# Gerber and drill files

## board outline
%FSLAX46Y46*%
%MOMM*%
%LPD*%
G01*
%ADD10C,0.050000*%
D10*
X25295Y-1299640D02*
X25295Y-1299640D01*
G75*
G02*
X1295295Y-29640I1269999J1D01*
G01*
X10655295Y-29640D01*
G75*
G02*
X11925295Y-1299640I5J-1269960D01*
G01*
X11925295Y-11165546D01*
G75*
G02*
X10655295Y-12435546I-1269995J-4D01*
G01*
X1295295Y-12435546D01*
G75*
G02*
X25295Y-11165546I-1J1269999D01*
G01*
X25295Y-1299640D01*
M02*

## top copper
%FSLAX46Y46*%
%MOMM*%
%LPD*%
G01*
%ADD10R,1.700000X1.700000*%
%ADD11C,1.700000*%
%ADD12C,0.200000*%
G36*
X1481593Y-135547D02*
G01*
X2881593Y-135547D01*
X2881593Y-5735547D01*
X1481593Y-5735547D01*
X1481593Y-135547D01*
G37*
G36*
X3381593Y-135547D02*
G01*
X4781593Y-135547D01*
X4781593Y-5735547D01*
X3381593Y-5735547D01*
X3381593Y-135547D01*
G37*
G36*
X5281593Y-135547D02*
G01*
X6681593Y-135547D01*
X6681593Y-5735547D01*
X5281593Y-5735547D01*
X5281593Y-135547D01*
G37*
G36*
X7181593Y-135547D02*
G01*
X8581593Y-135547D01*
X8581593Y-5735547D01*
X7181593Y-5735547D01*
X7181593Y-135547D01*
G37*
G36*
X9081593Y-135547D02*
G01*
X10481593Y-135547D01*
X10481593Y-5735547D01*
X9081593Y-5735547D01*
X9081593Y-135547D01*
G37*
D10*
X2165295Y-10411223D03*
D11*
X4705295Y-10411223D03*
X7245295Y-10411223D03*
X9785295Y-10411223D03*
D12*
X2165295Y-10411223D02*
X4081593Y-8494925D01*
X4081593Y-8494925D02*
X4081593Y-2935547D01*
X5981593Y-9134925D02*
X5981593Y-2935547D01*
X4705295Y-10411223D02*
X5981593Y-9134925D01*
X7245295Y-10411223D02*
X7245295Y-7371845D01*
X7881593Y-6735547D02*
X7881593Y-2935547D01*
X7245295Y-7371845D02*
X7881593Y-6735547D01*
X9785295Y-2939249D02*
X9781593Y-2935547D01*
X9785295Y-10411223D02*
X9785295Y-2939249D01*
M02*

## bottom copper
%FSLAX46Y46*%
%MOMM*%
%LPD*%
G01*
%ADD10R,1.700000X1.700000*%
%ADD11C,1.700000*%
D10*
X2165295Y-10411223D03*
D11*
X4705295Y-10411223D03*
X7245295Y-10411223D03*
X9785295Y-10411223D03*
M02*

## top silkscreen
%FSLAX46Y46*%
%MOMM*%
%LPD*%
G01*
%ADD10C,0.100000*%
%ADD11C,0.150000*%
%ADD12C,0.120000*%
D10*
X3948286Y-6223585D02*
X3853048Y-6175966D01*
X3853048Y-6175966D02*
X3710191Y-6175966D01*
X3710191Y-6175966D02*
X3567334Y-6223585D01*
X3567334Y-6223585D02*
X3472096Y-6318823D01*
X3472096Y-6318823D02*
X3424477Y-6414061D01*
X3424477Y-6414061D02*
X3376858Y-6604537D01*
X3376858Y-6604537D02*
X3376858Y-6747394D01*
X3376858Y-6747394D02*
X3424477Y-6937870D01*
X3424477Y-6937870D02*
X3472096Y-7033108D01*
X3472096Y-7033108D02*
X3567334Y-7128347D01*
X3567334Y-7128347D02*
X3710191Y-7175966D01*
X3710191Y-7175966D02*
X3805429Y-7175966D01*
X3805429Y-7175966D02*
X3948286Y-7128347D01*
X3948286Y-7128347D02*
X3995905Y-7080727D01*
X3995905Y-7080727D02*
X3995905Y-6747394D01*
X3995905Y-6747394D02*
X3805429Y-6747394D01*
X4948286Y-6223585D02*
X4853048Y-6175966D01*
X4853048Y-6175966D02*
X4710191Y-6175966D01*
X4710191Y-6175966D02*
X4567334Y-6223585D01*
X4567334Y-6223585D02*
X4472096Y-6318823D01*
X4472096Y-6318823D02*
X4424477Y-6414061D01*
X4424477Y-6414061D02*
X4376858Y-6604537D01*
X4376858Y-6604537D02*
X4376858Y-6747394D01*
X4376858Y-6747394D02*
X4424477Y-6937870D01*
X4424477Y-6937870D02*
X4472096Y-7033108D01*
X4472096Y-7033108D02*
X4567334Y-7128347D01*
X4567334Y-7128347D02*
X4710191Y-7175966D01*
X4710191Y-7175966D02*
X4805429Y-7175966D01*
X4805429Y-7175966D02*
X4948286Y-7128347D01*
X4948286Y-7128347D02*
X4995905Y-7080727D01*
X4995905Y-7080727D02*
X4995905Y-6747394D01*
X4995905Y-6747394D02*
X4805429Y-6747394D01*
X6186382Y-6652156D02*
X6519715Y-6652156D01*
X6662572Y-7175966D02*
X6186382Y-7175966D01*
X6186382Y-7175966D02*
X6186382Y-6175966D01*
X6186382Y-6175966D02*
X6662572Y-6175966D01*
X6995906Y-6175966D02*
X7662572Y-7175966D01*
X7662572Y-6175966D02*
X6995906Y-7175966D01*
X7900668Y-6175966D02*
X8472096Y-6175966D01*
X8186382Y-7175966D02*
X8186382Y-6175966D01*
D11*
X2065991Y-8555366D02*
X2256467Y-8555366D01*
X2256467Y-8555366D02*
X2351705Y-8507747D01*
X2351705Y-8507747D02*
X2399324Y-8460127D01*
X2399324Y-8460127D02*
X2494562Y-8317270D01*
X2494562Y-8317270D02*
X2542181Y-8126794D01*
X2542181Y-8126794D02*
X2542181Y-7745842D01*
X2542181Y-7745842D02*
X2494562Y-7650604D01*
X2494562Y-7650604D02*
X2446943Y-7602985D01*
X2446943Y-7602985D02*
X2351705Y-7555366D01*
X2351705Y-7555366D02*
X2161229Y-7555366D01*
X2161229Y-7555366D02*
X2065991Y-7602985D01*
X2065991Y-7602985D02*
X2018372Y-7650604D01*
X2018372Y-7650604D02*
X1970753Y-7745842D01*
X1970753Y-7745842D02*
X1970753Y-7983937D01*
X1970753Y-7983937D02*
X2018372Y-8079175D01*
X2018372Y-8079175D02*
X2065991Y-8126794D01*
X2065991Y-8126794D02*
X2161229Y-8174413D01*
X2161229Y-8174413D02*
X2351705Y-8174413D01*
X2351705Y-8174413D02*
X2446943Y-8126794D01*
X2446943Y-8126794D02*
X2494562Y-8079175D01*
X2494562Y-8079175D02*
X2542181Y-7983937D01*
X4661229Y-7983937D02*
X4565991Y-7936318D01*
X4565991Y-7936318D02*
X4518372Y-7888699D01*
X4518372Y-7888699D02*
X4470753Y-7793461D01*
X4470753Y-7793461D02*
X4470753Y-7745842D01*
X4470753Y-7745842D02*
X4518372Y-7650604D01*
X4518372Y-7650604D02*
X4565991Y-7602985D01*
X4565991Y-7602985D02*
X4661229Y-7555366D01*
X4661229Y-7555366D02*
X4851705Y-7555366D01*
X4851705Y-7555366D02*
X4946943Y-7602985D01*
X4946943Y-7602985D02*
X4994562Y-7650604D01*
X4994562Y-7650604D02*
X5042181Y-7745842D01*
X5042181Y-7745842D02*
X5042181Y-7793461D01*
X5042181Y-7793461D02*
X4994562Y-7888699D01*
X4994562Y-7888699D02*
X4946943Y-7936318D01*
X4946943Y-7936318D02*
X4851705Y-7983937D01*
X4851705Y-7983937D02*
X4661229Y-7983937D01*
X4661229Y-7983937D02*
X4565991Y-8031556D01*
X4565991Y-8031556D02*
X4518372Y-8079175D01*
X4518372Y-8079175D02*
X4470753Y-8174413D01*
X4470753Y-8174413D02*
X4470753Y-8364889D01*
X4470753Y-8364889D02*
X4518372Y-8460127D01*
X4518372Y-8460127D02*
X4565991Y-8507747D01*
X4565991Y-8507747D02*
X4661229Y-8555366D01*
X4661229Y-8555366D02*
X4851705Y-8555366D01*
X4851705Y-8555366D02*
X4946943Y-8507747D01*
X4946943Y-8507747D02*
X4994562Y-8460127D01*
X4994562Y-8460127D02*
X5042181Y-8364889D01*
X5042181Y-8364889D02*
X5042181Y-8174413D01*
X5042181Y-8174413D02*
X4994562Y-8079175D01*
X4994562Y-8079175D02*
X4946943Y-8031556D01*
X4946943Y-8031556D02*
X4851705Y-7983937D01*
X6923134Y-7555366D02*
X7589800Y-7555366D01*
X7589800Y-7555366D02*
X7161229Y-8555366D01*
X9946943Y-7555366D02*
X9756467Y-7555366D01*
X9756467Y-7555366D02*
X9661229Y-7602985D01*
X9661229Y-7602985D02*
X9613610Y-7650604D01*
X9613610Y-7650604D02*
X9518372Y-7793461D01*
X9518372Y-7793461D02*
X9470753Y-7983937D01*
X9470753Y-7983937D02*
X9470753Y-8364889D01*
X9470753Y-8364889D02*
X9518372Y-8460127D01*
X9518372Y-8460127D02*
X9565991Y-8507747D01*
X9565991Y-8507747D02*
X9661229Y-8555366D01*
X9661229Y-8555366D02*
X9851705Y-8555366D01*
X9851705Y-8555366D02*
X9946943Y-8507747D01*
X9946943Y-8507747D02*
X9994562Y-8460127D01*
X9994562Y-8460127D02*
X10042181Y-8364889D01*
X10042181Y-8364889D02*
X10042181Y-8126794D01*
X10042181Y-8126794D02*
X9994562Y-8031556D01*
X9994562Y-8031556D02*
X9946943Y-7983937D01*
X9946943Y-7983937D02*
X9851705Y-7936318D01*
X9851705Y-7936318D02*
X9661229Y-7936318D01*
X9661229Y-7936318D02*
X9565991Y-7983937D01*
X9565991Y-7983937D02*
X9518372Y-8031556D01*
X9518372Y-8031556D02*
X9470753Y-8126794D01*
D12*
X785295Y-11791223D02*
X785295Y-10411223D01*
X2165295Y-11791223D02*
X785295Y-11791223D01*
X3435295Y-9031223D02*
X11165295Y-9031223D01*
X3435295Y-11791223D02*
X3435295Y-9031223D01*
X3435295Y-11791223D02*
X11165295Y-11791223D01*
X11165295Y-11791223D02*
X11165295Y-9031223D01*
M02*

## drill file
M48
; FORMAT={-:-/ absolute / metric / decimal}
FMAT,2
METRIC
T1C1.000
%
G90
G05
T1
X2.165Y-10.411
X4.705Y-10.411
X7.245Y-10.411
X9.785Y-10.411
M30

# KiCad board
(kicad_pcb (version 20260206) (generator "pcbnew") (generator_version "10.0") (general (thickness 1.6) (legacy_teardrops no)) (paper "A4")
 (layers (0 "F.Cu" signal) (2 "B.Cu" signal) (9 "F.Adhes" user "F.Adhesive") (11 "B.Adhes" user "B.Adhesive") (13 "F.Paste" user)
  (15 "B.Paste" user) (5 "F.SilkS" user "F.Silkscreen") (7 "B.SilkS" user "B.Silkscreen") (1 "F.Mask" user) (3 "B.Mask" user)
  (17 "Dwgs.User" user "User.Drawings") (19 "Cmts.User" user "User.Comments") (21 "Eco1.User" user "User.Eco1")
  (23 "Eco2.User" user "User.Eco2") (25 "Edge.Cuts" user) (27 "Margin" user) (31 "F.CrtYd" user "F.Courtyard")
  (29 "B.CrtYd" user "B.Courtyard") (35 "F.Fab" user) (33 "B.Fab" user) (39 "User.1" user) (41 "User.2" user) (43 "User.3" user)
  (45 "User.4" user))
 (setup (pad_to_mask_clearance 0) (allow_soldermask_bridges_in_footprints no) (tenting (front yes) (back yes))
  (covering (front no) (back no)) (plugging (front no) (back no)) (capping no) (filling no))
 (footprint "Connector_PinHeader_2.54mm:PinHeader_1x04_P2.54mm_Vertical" (layer "F.Cu") (at 2.165295 10.411223 90)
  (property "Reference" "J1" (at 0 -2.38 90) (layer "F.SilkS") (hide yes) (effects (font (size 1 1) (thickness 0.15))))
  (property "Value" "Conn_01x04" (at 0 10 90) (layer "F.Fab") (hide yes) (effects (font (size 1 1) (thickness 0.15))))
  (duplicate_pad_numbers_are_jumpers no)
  (fp_line (start -1.38 -1.38) (end 0 -1.38) (stroke (width 0.12) (type solid)) (layer "F.SilkS"))
  (fp_line (start -1.38 0) (end -1.38 -1.38) (stroke (width 0.12) (type solid)) (layer "F.SilkS"))
  (fp_line (start 1.38 1.27) (end 1.38 9) (stroke (width 0.12) (type solid)) (layer "F.SilkS"))
  (fp_line (start -1.38 1.27) (end 1.38 1.27) (stroke (width 0.12) (type solid)) (layer "F.SilkS"))
  (fp_line (start -1.38 1.27) (end -1.38 9) (stroke (width 0.12) (type solid)) (layer "F.SilkS"))
  (fp_line (start -1.38 9) (end 1.38 9) (stroke (width 0.12) (type solid)) (layer "F.SilkS"))
  (pad "1" thru_hole rect (at 0 0 90) (size 1.7 1.7) (drill 1) (layers "*.Cu" "*.Mask") (remove_unused_layers no)
   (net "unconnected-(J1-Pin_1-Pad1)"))
  (pad "2" thru_hole circle (at 0 2.54 90) (size 1.7 1.7) (drill 1) (layers "*.Cu" "*.Mask") (remove_unused_layers no)
   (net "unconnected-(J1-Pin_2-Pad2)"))
  (pad "3" thru_hole circle (at 0 5.08 90) (size 1.7 1.7) (drill 1) (layers "*.Cu" "*.Mask") (remove_unused_layers no)
   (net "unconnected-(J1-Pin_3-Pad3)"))
  (pad "4" thru_hole circle (at 0 7.62 90) (size 1.7 1.7) (drill 1) (layers "*.Cu" "*.Mask") (remove_unused_layers no)
   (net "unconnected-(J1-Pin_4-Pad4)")))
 (gr_rect (start 1.481593 0.135547) (end 2.881593 5.735547) (stroke (width 0) (type solid)) (fill yes) (layers "F.Cu" "F.Mask"))
 (gr_rect (start 3.381593 0.135547) (end 4.781593 5.735547) (stroke (width 0) (type solid)) (fill yes) (layers "F.Cu" "F.Mask")
  (net "unconnected-(J1-Pin_1-Pad1)"))
 (gr_rect (start 5.281593 0.135547) (end 6.681593 5.735547) (stroke (width 0) (type solid)) (fill yes) (layers "F.Cu" "F.Mask")
  (net "unconnected-(J1-Pin_2-Pad2)"))
 (gr_rect (start 7.181593 0.135547) (end 8.581593 5.735547) (stroke (width 0) (type solid)) (fill yes) (layers "F.Cu" "F.Mask")
  (net "unconnected-(J1-Pin_3-Pad3)"))
 (gr_rect (start 9.081593 0.135547) (end 10.481593 5.735547) (stroke (width 0) (type solid)) (fill yes) (layers "F.Cu" "F.Mask")
  (net "unconnected-(J1-Pin_4-Pad4)"))
 (gr_rect (start 0.025295 0.02964) (end 11.925295 12.435546) (radius 1.27) (stroke (width 0.05) (type solid)) (fill no) (layer "Edge.Cuts"))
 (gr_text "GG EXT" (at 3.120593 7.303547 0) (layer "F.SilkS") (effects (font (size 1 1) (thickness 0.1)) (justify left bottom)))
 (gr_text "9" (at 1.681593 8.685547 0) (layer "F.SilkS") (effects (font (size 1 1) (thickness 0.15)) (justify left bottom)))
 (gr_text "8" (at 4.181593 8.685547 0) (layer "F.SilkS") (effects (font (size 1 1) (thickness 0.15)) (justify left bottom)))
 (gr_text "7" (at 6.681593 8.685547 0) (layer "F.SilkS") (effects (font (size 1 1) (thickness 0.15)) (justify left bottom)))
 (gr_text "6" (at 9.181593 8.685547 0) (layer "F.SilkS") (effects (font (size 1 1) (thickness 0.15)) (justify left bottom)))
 (segment (start 2.165295 10.411223) (end 4.081593 8.494925) (width 0.2) (layer "F.Cu") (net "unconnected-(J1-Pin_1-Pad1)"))
 (segment (start 4.081593 8.494925) (end 4.081593 2.935547) (width 0.2) (layer "F.Cu") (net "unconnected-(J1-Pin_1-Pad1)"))
 (segment (start 5.981593 9.134925) (end 5.981593 2.935547) (width 0.2) (layer "F.Cu") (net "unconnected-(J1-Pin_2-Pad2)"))
 (segment (start 4.705295 10.411223) (end 5.981593 9.134925) (width 0.2) (layer "F.Cu") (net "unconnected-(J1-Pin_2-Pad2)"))
 (segment (start 7.245295 10.411223) (end 7.245295 7.371845) (width 0.2) (layer "F.Cu") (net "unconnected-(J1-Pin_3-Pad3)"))
 (segment (start 7.881593 6.735547) (end 7.881593 2.935547) (width 0.2) (layer "F.Cu") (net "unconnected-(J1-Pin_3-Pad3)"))
 (segment (start 7.245295 7.371845) (end 7.881593 6.735547) (width 0.2) (layer "F.Cu") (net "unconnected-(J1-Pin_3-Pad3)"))
 (segment (start 9.785295 2.939249) (end 9.781593 2.935547) (width 0.2) (layer "F.Cu") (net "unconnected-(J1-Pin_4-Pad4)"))
 (segment (start 9.785295 10.411223) (end 9.785295 2.939249) (width 0.2) (layer "F.Cu") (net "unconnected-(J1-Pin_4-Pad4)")))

